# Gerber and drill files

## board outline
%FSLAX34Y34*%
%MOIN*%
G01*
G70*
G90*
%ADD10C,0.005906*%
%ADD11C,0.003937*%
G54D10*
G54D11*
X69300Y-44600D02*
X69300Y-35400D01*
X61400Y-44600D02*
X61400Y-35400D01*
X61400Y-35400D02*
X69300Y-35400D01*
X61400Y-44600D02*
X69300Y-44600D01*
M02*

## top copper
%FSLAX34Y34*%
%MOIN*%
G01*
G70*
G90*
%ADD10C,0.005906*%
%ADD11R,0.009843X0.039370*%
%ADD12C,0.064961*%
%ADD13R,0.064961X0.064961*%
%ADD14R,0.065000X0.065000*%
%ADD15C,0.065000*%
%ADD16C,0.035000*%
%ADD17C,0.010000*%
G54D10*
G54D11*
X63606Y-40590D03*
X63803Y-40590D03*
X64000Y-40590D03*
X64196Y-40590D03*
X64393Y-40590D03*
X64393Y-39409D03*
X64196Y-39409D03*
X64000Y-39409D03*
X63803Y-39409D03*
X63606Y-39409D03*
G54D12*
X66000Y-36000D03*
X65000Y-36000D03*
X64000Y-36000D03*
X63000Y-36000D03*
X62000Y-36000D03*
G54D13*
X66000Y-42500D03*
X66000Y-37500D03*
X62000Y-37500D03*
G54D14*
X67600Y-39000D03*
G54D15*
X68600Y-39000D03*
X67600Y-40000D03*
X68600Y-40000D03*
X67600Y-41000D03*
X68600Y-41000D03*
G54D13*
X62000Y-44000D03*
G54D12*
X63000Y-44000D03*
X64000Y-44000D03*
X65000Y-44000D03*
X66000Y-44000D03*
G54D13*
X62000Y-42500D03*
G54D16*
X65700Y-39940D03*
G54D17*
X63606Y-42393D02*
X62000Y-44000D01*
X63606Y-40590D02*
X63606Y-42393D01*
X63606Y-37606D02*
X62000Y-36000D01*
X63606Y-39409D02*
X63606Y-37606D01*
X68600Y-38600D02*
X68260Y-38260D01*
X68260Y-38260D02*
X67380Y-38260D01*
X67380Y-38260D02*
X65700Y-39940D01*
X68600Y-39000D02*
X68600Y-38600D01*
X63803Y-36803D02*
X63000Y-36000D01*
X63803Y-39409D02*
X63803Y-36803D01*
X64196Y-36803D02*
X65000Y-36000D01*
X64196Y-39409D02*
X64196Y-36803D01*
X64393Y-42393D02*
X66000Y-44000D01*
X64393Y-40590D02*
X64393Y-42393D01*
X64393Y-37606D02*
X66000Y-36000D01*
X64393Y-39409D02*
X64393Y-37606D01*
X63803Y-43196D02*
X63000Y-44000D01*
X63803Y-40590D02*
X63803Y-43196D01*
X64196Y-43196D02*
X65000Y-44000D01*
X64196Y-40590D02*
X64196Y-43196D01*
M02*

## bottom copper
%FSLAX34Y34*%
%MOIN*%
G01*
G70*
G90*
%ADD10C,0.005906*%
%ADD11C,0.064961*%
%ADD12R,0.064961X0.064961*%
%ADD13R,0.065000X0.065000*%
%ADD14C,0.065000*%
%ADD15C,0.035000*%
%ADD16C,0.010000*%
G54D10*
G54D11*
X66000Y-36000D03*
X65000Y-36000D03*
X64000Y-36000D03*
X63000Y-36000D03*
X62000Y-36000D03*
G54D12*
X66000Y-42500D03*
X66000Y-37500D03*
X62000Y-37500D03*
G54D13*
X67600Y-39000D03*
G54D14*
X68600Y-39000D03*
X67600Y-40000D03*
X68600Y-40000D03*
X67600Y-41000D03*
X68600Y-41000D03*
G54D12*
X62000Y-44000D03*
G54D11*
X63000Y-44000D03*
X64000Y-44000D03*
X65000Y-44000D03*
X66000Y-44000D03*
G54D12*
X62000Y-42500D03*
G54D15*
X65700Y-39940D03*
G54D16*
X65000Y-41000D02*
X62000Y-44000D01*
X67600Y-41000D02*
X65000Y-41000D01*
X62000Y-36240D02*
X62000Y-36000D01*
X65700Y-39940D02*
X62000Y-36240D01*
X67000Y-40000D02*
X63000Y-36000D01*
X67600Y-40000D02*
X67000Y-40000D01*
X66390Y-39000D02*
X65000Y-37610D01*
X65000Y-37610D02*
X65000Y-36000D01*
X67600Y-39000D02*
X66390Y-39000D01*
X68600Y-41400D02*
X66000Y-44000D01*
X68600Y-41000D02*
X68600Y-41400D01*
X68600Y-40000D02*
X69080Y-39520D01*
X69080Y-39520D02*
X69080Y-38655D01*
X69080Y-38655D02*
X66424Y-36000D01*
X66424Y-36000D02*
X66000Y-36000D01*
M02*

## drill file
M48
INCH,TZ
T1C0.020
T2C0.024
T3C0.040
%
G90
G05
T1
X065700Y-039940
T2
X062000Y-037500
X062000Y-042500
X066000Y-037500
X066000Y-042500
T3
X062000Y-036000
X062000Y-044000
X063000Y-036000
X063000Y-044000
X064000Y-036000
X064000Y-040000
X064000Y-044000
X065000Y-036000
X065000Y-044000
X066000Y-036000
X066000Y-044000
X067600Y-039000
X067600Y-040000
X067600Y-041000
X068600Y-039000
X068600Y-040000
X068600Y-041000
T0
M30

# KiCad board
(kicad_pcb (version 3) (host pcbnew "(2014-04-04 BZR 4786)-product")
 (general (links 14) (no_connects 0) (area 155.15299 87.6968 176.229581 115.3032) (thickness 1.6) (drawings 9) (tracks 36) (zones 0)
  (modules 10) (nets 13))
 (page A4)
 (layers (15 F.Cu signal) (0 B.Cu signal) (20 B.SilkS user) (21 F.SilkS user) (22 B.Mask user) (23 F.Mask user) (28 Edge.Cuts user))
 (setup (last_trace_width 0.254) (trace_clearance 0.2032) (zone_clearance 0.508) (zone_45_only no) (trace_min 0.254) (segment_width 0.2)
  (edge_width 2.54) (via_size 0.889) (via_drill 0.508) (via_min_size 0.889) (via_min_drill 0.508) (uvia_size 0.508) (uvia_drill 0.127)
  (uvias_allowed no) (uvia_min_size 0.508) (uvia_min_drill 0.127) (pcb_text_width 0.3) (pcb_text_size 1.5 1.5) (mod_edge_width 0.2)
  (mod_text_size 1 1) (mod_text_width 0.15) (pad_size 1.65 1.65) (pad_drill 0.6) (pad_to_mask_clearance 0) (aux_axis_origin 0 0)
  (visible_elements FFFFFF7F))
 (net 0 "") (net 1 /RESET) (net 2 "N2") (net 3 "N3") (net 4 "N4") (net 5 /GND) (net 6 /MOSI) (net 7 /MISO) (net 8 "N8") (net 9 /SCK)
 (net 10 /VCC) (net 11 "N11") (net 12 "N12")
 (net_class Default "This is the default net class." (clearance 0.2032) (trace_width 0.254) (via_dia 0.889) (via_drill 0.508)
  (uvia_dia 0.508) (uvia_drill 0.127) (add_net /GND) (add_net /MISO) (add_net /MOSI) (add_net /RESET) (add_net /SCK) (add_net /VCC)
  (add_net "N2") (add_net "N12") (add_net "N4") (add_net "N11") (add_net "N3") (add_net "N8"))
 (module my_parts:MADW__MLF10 (layer F.Cu) (at 162.56 101.6 90)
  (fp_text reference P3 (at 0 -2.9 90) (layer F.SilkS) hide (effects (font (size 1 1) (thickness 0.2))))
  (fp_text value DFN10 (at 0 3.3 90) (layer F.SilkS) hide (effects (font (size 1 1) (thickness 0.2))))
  (pad 1 smd rect (at -1.5 -1 90) (size 1 0.25) (layers F.Cu F.Mask) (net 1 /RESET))
  (pad 2 smd rect (at -1.5 -0.5 90) (size 1 0.25) (layers F.Cu F.Mask) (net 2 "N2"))
  (pad 3 smd rect (at -1.5 0 90) (size 1 0.25) (layers F.Cu F.Mask) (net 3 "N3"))
  (pad 4 smd rect (at -1.5 0.5 90) (size 1 0.25) (layers F.Cu F.Mask) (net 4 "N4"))
  (pad 5 smd rect (at -1.5 1 90) (size 1 0.25) (layers F.Cu F.Mask) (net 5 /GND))
  (pad 6 smd rect (at 1.5 1 90) (size 1 0.25) (layers F.Cu F.Mask) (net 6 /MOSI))
  (pad 7 smd rect (at 1.5 0.5 90) (size 1 0.25) (layers F.Cu F.Mask) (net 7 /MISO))
  (pad 8 smd rect (at 1.5 0 90) (size 1 0.25) (layers F.Cu F.Mask) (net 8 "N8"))
  (pad 9 smd rect (at 1.5 -0.5 90) (size 1 0.25) (layers F.Cu F.Mask) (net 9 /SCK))
  (pad 10 smd rect (at 1.5 -1 90) (size 1 0.25) (layers F.Cu F.Mask) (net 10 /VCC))
  (pad "" np_thru_hole circle (at 0 0 90) (size 1.016 1.016) (drill 1.016) (layers *.Cu *.Mask F.SilkS)))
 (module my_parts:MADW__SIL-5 (layer F.Cu) (at 162.56 91.44 180)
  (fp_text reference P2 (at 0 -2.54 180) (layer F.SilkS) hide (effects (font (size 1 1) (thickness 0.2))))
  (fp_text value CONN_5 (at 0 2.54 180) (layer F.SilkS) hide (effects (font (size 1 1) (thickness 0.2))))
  (pad 1 thru_hole circle (at -5.08 0 180) (size 1.65 1.65) (drill 1.016) (layers *.Cu *.Mask F.SilkS) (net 6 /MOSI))
  (pad 2 thru_hole circle (at -2.54 0 180) (size 1.65 1.65) (drill 1.016) (layers *.Cu *.Mask F.SilkS) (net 7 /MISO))
  (pad 3 thru_hole circle (at 0 0 180) (size 1.65 1.65) (drill 1.016) (layers *.Cu *.Mask F.SilkS) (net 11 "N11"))
  (pad 4 thru_hole circle (at 2.54 0 180) (size 1.65 1.65) (drill 1.016) (layers *.Cu *.Mask F.SilkS) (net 9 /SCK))
  (pad 5 thru_hole circle (at 5.08 0 180) (size 1.65 1.65) (drill 1.016) (layers *.Cu *.Mask F.SilkS) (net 10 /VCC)))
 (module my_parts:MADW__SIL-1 (layer F.Cu) (at 167.64 107.95)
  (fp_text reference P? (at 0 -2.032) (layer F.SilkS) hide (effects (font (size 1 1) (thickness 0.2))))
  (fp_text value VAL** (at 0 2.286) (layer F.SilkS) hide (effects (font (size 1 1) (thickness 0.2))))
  (pad 1 thru_hole rect (at 0 0) (size 1.65 1.65) (drill 0.6) (layers *.Cu *.Mask F.SilkS)))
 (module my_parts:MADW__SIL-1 (layer F.Cu) (at 167.64 95.25)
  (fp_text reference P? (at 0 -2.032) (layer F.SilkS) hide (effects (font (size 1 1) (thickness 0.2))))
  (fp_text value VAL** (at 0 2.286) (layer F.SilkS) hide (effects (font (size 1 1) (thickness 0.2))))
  (pad 1 thru_hole rect (at 0 0) (size 1.65 1.65) (drill 0.6) (layers *.Cu *.Mask F.SilkS)))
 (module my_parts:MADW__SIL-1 (layer F.Cu) (at 157.48 95.25)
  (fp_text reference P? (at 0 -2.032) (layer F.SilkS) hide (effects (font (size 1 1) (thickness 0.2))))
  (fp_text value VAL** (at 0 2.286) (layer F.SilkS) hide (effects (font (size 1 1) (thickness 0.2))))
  (pad 1 thru_hole rect (at 0 0) (size 1.65 1.65) (drill 0.6) (layers *.Cu *.Mask F.SilkS)))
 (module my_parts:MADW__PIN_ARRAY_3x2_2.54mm (layer F.Cu) (at 172.974 101.6 90)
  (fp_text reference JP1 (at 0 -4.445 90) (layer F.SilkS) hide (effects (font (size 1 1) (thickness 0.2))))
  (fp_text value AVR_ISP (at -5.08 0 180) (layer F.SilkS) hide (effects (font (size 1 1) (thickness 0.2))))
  (pad 1 thru_hole rect (at 2.54 -1.27 90) (size 1.651 1.651) (drill 1.016) (layers *.Cu *.Mask F.SilkS) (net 7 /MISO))
  (pad 2 thru_hole circle (at 2.54 1.27 90) (size 1.651 1.651) (drill 1.016) (layers *.Cu *.Mask F.SilkS) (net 10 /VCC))
  (pad 3 thru_hole circle (at 0 -1.27 90) (size 1.651 1.651) (drill 1.016) (layers *.Cu *.Mask F.SilkS) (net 9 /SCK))
  (pad 4 thru_hole circle (at 0 1.27 90) (size 1.651 1.651) (drill 1.016) (layers *.Cu *.Mask F.SilkS) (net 6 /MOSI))
  (pad 5 thru_hole circle (at -2.54 -1.27 90) (size 1.651 1.651) (drill 1.016) (layers *.Cu *.Mask F.SilkS) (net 1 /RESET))
  (pad 6 thru_hole circle (at -2.54 1.27 90) (size 1.651 1.651) (drill 1.016) (layers *.Cu *.Mask F.SilkS) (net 5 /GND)))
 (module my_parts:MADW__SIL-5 (layer F.Cu) (at 162.56 111.76)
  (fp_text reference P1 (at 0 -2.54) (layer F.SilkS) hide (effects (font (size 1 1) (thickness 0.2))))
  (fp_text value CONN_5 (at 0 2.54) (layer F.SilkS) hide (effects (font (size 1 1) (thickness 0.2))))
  (pad 1 thru_hole rect (at -5.08 0) (size 1.65 1.65) (drill 1.016) (layers *.Cu *.Mask F.SilkS) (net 1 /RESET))
  (pad 2 thru_hole circle (at -2.54 0) (size 1.65 1.65) (drill 1.016) (layers *.Cu *.Mask F.SilkS) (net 2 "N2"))
  (pad 3 thru_hole circle (at 0 0) (size 1.65 1.65) (drill 1.016) (layers *.Cu *.Mask F.SilkS) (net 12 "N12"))
  (pad 4 thru_hole circle (at 2.54 0) (size 1.65 1.65) (drill 1.016) (layers *.Cu *.Mask F.SilkS) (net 4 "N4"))
  (pad 5 thru_hole circle (at 5.08 0) (size 1.65 1.65) (drill 1.016) (layers *.Cu *.Mask F.SilkS) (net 5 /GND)))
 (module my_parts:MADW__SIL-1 (layer F.Cu) (at 157.48 107.95)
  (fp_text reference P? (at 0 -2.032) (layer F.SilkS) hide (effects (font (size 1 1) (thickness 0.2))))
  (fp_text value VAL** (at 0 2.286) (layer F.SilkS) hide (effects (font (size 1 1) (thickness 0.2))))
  (pad 1 thru_hole rect (at 0 0) (size 1.65 1.65) (drill 0.6) (layers *.Cu *.Mask F.SilkS)))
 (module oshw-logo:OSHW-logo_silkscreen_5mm (layer F.Cu) (at 172.72 110.2614 90)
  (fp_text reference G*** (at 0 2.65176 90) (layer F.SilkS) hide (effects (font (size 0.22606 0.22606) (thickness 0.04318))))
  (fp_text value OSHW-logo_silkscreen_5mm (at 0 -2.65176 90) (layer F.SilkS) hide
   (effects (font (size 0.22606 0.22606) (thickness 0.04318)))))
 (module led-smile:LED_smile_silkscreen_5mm (layer F.Cu) (at 172.8216 93.345 90)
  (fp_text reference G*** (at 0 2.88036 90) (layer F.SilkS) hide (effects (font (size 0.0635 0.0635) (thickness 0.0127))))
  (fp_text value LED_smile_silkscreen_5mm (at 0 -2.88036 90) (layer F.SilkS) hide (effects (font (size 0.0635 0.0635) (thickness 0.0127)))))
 (gr_line (start 176.022 113.284) (end 176.022 89.916) (angle 90) (layer Edge.Cuts) (width 0.1))
 (gr_line (start 155.956 113.284) (end 155.956 89.916) (angle 90) (layer Edge.Cuts) (width 0.1))
 (gr_line (start 155.956 89.916) (end 176.022 89.916) (angle 90) (layer Edge.Cuts) (width 0.1))
 (gr_line (start 155.956 113.284) (end 176.022 113.284) (angle 90) (layer Edge.Cuts) (width 0.1))
 (segment (start 161.56 107.68) (end 157.48 111.76) (width 0.254) (layer F.Cu) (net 1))
 (segment (start 161.56 103.1) (end 161.56 107.68) (width 0.254) (layer F.Cu) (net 1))
 (segment (start 165.1 104.14) (end 157.48 111.76) (width 0.254) (layer B.Cu) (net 1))
 (segment (start 171.704 104.14) (end 165.1 104.14) (width 0.254) (layer B.Cu) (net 1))
 (segment (start 161.56 95.52) (end 157.48 91.44) (width 0.254) (layer F.Cu) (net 10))
 (segment (start 161.56 100.1) (end 161.56 95.52) (width 0.254) (layer F.Cu) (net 10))
 (segment (start 157.48 92.0496) (end 157.48 91.44) (width 0.254) (layer B.Cu) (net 10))
 (segment (start 174.244 98.044) (end 173.3804 97.1804) (width 0.254) (layer F.Cu) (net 10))
 (segment (start 173.3804 97.1804) (end 171.1452 97.1804) (width 0.254) (layer F.Cu) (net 10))
 (segment (start 171.1452 97.1804) (end 166.878 101.4476) (width 0.254) (layer F.Cu) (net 10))
 (via (at 166.878 101.4476) (size 0.889) (layers F.Cu B.Cu) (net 10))
 (segment (start 166.878 101.4476) (end 157.48 92.0496) (width 0.254) (layer B.Cu) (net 10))
 (segment (start 174.244 99.06) (end 174.244 98.044) (width 0.254) (layer F.Cu) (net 10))
 (segment (start 162.06 93.48) (end 160.02 91.44) (width 0.254) (layer F.Cu) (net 9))
 (segment (start 162.06 100.1) (end 162.06 93.48) (width 0.254) (layer F.Cu) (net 9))
 (segment (start 170.18 101.6) (end 160.02 91.44) (width 0.254) (layer B.Cu) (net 9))
 (segment (start 171.704 101.6) (end 170.18 101.6) (width 0.254) (layer B.Cu) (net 9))
 (segment (start 163.06 93.48) (end 165.1 91.44) (width 0.254) (layer F.Cu) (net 7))
 (segment (start 163.06 100.1) (end 163.06 93.48) (width 0.254) (layer F.Cu) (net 7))
 (segment (start 168.6306 99.06) (end 165.1 95.5294) (width 0.254) (layer B.Cu) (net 7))
 (segment (start 165.1 95.5294) (end 165.1 91.44) (width 0.254) (layer B.Cu) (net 7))
 (segment (start 171.704 99.06) (end 168.6306 99.06) (width 0.254) (layer B.Cu) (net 7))
 (segment (start 163.56 107.68) (end 167.64 111.76) (width 0.254) (layer F.Cu) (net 5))
 (segment (start 163.56 103.1) (end 163.56 107.68) (width 0.254) (layer F.Cu) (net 5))
 (segment (start 174.244 105.156) (end 167.64 111.76) (width 0.254) (layer B.Cu) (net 5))
 (segment (start 174.244 104.14) (end 174.244 105.156) (width 0.254) (layer B.Cu) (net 5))
 (segment (start 163.56 95.52) (end 167.64 91.44) (width 0.254) (layer F.Cu) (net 6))
 (segment (start 163.56 100.1) (end 163.56 95.52) (width 0.254) (layer F.Cu) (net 6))
 (segment (start 174.244 101.6) (end 175.4632 100.3808) (width 0.254) (layer B.Cu) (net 6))
 (segment (start 175.4632 100.3808) (end 175.4632 98.1842) (width 0.254) (layer B.Cu) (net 6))
 (segment (start 175.4632 98.1842) (end 168.719 91.44) (width 0.254) (layer B.Cu) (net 6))
 (segment (start 168.719 91.44) (end 167.64 91.44) (width 0.254) (layer B.Cu) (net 6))
 (segment (start 162.06 109.72) (end 160.02 111.76) (width 0.254) (layer F.Cu) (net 2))
 (segment (start 162.06 103.1) (end 162.06 109.72) (width 0.254) (layer F.Cu) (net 2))
 (segment (start 163.06 109.72) (end 165.1 111.76) (width 0.254) (layer F.Cu) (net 4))
 (segment (start 163.06 103.1) (end 163.06 109.72) (width 0.254) (layer F.Cu) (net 4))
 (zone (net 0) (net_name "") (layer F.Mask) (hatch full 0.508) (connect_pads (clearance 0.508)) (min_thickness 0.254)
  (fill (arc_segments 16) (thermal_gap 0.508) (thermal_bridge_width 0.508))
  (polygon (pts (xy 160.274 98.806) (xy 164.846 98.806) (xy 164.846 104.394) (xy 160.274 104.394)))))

